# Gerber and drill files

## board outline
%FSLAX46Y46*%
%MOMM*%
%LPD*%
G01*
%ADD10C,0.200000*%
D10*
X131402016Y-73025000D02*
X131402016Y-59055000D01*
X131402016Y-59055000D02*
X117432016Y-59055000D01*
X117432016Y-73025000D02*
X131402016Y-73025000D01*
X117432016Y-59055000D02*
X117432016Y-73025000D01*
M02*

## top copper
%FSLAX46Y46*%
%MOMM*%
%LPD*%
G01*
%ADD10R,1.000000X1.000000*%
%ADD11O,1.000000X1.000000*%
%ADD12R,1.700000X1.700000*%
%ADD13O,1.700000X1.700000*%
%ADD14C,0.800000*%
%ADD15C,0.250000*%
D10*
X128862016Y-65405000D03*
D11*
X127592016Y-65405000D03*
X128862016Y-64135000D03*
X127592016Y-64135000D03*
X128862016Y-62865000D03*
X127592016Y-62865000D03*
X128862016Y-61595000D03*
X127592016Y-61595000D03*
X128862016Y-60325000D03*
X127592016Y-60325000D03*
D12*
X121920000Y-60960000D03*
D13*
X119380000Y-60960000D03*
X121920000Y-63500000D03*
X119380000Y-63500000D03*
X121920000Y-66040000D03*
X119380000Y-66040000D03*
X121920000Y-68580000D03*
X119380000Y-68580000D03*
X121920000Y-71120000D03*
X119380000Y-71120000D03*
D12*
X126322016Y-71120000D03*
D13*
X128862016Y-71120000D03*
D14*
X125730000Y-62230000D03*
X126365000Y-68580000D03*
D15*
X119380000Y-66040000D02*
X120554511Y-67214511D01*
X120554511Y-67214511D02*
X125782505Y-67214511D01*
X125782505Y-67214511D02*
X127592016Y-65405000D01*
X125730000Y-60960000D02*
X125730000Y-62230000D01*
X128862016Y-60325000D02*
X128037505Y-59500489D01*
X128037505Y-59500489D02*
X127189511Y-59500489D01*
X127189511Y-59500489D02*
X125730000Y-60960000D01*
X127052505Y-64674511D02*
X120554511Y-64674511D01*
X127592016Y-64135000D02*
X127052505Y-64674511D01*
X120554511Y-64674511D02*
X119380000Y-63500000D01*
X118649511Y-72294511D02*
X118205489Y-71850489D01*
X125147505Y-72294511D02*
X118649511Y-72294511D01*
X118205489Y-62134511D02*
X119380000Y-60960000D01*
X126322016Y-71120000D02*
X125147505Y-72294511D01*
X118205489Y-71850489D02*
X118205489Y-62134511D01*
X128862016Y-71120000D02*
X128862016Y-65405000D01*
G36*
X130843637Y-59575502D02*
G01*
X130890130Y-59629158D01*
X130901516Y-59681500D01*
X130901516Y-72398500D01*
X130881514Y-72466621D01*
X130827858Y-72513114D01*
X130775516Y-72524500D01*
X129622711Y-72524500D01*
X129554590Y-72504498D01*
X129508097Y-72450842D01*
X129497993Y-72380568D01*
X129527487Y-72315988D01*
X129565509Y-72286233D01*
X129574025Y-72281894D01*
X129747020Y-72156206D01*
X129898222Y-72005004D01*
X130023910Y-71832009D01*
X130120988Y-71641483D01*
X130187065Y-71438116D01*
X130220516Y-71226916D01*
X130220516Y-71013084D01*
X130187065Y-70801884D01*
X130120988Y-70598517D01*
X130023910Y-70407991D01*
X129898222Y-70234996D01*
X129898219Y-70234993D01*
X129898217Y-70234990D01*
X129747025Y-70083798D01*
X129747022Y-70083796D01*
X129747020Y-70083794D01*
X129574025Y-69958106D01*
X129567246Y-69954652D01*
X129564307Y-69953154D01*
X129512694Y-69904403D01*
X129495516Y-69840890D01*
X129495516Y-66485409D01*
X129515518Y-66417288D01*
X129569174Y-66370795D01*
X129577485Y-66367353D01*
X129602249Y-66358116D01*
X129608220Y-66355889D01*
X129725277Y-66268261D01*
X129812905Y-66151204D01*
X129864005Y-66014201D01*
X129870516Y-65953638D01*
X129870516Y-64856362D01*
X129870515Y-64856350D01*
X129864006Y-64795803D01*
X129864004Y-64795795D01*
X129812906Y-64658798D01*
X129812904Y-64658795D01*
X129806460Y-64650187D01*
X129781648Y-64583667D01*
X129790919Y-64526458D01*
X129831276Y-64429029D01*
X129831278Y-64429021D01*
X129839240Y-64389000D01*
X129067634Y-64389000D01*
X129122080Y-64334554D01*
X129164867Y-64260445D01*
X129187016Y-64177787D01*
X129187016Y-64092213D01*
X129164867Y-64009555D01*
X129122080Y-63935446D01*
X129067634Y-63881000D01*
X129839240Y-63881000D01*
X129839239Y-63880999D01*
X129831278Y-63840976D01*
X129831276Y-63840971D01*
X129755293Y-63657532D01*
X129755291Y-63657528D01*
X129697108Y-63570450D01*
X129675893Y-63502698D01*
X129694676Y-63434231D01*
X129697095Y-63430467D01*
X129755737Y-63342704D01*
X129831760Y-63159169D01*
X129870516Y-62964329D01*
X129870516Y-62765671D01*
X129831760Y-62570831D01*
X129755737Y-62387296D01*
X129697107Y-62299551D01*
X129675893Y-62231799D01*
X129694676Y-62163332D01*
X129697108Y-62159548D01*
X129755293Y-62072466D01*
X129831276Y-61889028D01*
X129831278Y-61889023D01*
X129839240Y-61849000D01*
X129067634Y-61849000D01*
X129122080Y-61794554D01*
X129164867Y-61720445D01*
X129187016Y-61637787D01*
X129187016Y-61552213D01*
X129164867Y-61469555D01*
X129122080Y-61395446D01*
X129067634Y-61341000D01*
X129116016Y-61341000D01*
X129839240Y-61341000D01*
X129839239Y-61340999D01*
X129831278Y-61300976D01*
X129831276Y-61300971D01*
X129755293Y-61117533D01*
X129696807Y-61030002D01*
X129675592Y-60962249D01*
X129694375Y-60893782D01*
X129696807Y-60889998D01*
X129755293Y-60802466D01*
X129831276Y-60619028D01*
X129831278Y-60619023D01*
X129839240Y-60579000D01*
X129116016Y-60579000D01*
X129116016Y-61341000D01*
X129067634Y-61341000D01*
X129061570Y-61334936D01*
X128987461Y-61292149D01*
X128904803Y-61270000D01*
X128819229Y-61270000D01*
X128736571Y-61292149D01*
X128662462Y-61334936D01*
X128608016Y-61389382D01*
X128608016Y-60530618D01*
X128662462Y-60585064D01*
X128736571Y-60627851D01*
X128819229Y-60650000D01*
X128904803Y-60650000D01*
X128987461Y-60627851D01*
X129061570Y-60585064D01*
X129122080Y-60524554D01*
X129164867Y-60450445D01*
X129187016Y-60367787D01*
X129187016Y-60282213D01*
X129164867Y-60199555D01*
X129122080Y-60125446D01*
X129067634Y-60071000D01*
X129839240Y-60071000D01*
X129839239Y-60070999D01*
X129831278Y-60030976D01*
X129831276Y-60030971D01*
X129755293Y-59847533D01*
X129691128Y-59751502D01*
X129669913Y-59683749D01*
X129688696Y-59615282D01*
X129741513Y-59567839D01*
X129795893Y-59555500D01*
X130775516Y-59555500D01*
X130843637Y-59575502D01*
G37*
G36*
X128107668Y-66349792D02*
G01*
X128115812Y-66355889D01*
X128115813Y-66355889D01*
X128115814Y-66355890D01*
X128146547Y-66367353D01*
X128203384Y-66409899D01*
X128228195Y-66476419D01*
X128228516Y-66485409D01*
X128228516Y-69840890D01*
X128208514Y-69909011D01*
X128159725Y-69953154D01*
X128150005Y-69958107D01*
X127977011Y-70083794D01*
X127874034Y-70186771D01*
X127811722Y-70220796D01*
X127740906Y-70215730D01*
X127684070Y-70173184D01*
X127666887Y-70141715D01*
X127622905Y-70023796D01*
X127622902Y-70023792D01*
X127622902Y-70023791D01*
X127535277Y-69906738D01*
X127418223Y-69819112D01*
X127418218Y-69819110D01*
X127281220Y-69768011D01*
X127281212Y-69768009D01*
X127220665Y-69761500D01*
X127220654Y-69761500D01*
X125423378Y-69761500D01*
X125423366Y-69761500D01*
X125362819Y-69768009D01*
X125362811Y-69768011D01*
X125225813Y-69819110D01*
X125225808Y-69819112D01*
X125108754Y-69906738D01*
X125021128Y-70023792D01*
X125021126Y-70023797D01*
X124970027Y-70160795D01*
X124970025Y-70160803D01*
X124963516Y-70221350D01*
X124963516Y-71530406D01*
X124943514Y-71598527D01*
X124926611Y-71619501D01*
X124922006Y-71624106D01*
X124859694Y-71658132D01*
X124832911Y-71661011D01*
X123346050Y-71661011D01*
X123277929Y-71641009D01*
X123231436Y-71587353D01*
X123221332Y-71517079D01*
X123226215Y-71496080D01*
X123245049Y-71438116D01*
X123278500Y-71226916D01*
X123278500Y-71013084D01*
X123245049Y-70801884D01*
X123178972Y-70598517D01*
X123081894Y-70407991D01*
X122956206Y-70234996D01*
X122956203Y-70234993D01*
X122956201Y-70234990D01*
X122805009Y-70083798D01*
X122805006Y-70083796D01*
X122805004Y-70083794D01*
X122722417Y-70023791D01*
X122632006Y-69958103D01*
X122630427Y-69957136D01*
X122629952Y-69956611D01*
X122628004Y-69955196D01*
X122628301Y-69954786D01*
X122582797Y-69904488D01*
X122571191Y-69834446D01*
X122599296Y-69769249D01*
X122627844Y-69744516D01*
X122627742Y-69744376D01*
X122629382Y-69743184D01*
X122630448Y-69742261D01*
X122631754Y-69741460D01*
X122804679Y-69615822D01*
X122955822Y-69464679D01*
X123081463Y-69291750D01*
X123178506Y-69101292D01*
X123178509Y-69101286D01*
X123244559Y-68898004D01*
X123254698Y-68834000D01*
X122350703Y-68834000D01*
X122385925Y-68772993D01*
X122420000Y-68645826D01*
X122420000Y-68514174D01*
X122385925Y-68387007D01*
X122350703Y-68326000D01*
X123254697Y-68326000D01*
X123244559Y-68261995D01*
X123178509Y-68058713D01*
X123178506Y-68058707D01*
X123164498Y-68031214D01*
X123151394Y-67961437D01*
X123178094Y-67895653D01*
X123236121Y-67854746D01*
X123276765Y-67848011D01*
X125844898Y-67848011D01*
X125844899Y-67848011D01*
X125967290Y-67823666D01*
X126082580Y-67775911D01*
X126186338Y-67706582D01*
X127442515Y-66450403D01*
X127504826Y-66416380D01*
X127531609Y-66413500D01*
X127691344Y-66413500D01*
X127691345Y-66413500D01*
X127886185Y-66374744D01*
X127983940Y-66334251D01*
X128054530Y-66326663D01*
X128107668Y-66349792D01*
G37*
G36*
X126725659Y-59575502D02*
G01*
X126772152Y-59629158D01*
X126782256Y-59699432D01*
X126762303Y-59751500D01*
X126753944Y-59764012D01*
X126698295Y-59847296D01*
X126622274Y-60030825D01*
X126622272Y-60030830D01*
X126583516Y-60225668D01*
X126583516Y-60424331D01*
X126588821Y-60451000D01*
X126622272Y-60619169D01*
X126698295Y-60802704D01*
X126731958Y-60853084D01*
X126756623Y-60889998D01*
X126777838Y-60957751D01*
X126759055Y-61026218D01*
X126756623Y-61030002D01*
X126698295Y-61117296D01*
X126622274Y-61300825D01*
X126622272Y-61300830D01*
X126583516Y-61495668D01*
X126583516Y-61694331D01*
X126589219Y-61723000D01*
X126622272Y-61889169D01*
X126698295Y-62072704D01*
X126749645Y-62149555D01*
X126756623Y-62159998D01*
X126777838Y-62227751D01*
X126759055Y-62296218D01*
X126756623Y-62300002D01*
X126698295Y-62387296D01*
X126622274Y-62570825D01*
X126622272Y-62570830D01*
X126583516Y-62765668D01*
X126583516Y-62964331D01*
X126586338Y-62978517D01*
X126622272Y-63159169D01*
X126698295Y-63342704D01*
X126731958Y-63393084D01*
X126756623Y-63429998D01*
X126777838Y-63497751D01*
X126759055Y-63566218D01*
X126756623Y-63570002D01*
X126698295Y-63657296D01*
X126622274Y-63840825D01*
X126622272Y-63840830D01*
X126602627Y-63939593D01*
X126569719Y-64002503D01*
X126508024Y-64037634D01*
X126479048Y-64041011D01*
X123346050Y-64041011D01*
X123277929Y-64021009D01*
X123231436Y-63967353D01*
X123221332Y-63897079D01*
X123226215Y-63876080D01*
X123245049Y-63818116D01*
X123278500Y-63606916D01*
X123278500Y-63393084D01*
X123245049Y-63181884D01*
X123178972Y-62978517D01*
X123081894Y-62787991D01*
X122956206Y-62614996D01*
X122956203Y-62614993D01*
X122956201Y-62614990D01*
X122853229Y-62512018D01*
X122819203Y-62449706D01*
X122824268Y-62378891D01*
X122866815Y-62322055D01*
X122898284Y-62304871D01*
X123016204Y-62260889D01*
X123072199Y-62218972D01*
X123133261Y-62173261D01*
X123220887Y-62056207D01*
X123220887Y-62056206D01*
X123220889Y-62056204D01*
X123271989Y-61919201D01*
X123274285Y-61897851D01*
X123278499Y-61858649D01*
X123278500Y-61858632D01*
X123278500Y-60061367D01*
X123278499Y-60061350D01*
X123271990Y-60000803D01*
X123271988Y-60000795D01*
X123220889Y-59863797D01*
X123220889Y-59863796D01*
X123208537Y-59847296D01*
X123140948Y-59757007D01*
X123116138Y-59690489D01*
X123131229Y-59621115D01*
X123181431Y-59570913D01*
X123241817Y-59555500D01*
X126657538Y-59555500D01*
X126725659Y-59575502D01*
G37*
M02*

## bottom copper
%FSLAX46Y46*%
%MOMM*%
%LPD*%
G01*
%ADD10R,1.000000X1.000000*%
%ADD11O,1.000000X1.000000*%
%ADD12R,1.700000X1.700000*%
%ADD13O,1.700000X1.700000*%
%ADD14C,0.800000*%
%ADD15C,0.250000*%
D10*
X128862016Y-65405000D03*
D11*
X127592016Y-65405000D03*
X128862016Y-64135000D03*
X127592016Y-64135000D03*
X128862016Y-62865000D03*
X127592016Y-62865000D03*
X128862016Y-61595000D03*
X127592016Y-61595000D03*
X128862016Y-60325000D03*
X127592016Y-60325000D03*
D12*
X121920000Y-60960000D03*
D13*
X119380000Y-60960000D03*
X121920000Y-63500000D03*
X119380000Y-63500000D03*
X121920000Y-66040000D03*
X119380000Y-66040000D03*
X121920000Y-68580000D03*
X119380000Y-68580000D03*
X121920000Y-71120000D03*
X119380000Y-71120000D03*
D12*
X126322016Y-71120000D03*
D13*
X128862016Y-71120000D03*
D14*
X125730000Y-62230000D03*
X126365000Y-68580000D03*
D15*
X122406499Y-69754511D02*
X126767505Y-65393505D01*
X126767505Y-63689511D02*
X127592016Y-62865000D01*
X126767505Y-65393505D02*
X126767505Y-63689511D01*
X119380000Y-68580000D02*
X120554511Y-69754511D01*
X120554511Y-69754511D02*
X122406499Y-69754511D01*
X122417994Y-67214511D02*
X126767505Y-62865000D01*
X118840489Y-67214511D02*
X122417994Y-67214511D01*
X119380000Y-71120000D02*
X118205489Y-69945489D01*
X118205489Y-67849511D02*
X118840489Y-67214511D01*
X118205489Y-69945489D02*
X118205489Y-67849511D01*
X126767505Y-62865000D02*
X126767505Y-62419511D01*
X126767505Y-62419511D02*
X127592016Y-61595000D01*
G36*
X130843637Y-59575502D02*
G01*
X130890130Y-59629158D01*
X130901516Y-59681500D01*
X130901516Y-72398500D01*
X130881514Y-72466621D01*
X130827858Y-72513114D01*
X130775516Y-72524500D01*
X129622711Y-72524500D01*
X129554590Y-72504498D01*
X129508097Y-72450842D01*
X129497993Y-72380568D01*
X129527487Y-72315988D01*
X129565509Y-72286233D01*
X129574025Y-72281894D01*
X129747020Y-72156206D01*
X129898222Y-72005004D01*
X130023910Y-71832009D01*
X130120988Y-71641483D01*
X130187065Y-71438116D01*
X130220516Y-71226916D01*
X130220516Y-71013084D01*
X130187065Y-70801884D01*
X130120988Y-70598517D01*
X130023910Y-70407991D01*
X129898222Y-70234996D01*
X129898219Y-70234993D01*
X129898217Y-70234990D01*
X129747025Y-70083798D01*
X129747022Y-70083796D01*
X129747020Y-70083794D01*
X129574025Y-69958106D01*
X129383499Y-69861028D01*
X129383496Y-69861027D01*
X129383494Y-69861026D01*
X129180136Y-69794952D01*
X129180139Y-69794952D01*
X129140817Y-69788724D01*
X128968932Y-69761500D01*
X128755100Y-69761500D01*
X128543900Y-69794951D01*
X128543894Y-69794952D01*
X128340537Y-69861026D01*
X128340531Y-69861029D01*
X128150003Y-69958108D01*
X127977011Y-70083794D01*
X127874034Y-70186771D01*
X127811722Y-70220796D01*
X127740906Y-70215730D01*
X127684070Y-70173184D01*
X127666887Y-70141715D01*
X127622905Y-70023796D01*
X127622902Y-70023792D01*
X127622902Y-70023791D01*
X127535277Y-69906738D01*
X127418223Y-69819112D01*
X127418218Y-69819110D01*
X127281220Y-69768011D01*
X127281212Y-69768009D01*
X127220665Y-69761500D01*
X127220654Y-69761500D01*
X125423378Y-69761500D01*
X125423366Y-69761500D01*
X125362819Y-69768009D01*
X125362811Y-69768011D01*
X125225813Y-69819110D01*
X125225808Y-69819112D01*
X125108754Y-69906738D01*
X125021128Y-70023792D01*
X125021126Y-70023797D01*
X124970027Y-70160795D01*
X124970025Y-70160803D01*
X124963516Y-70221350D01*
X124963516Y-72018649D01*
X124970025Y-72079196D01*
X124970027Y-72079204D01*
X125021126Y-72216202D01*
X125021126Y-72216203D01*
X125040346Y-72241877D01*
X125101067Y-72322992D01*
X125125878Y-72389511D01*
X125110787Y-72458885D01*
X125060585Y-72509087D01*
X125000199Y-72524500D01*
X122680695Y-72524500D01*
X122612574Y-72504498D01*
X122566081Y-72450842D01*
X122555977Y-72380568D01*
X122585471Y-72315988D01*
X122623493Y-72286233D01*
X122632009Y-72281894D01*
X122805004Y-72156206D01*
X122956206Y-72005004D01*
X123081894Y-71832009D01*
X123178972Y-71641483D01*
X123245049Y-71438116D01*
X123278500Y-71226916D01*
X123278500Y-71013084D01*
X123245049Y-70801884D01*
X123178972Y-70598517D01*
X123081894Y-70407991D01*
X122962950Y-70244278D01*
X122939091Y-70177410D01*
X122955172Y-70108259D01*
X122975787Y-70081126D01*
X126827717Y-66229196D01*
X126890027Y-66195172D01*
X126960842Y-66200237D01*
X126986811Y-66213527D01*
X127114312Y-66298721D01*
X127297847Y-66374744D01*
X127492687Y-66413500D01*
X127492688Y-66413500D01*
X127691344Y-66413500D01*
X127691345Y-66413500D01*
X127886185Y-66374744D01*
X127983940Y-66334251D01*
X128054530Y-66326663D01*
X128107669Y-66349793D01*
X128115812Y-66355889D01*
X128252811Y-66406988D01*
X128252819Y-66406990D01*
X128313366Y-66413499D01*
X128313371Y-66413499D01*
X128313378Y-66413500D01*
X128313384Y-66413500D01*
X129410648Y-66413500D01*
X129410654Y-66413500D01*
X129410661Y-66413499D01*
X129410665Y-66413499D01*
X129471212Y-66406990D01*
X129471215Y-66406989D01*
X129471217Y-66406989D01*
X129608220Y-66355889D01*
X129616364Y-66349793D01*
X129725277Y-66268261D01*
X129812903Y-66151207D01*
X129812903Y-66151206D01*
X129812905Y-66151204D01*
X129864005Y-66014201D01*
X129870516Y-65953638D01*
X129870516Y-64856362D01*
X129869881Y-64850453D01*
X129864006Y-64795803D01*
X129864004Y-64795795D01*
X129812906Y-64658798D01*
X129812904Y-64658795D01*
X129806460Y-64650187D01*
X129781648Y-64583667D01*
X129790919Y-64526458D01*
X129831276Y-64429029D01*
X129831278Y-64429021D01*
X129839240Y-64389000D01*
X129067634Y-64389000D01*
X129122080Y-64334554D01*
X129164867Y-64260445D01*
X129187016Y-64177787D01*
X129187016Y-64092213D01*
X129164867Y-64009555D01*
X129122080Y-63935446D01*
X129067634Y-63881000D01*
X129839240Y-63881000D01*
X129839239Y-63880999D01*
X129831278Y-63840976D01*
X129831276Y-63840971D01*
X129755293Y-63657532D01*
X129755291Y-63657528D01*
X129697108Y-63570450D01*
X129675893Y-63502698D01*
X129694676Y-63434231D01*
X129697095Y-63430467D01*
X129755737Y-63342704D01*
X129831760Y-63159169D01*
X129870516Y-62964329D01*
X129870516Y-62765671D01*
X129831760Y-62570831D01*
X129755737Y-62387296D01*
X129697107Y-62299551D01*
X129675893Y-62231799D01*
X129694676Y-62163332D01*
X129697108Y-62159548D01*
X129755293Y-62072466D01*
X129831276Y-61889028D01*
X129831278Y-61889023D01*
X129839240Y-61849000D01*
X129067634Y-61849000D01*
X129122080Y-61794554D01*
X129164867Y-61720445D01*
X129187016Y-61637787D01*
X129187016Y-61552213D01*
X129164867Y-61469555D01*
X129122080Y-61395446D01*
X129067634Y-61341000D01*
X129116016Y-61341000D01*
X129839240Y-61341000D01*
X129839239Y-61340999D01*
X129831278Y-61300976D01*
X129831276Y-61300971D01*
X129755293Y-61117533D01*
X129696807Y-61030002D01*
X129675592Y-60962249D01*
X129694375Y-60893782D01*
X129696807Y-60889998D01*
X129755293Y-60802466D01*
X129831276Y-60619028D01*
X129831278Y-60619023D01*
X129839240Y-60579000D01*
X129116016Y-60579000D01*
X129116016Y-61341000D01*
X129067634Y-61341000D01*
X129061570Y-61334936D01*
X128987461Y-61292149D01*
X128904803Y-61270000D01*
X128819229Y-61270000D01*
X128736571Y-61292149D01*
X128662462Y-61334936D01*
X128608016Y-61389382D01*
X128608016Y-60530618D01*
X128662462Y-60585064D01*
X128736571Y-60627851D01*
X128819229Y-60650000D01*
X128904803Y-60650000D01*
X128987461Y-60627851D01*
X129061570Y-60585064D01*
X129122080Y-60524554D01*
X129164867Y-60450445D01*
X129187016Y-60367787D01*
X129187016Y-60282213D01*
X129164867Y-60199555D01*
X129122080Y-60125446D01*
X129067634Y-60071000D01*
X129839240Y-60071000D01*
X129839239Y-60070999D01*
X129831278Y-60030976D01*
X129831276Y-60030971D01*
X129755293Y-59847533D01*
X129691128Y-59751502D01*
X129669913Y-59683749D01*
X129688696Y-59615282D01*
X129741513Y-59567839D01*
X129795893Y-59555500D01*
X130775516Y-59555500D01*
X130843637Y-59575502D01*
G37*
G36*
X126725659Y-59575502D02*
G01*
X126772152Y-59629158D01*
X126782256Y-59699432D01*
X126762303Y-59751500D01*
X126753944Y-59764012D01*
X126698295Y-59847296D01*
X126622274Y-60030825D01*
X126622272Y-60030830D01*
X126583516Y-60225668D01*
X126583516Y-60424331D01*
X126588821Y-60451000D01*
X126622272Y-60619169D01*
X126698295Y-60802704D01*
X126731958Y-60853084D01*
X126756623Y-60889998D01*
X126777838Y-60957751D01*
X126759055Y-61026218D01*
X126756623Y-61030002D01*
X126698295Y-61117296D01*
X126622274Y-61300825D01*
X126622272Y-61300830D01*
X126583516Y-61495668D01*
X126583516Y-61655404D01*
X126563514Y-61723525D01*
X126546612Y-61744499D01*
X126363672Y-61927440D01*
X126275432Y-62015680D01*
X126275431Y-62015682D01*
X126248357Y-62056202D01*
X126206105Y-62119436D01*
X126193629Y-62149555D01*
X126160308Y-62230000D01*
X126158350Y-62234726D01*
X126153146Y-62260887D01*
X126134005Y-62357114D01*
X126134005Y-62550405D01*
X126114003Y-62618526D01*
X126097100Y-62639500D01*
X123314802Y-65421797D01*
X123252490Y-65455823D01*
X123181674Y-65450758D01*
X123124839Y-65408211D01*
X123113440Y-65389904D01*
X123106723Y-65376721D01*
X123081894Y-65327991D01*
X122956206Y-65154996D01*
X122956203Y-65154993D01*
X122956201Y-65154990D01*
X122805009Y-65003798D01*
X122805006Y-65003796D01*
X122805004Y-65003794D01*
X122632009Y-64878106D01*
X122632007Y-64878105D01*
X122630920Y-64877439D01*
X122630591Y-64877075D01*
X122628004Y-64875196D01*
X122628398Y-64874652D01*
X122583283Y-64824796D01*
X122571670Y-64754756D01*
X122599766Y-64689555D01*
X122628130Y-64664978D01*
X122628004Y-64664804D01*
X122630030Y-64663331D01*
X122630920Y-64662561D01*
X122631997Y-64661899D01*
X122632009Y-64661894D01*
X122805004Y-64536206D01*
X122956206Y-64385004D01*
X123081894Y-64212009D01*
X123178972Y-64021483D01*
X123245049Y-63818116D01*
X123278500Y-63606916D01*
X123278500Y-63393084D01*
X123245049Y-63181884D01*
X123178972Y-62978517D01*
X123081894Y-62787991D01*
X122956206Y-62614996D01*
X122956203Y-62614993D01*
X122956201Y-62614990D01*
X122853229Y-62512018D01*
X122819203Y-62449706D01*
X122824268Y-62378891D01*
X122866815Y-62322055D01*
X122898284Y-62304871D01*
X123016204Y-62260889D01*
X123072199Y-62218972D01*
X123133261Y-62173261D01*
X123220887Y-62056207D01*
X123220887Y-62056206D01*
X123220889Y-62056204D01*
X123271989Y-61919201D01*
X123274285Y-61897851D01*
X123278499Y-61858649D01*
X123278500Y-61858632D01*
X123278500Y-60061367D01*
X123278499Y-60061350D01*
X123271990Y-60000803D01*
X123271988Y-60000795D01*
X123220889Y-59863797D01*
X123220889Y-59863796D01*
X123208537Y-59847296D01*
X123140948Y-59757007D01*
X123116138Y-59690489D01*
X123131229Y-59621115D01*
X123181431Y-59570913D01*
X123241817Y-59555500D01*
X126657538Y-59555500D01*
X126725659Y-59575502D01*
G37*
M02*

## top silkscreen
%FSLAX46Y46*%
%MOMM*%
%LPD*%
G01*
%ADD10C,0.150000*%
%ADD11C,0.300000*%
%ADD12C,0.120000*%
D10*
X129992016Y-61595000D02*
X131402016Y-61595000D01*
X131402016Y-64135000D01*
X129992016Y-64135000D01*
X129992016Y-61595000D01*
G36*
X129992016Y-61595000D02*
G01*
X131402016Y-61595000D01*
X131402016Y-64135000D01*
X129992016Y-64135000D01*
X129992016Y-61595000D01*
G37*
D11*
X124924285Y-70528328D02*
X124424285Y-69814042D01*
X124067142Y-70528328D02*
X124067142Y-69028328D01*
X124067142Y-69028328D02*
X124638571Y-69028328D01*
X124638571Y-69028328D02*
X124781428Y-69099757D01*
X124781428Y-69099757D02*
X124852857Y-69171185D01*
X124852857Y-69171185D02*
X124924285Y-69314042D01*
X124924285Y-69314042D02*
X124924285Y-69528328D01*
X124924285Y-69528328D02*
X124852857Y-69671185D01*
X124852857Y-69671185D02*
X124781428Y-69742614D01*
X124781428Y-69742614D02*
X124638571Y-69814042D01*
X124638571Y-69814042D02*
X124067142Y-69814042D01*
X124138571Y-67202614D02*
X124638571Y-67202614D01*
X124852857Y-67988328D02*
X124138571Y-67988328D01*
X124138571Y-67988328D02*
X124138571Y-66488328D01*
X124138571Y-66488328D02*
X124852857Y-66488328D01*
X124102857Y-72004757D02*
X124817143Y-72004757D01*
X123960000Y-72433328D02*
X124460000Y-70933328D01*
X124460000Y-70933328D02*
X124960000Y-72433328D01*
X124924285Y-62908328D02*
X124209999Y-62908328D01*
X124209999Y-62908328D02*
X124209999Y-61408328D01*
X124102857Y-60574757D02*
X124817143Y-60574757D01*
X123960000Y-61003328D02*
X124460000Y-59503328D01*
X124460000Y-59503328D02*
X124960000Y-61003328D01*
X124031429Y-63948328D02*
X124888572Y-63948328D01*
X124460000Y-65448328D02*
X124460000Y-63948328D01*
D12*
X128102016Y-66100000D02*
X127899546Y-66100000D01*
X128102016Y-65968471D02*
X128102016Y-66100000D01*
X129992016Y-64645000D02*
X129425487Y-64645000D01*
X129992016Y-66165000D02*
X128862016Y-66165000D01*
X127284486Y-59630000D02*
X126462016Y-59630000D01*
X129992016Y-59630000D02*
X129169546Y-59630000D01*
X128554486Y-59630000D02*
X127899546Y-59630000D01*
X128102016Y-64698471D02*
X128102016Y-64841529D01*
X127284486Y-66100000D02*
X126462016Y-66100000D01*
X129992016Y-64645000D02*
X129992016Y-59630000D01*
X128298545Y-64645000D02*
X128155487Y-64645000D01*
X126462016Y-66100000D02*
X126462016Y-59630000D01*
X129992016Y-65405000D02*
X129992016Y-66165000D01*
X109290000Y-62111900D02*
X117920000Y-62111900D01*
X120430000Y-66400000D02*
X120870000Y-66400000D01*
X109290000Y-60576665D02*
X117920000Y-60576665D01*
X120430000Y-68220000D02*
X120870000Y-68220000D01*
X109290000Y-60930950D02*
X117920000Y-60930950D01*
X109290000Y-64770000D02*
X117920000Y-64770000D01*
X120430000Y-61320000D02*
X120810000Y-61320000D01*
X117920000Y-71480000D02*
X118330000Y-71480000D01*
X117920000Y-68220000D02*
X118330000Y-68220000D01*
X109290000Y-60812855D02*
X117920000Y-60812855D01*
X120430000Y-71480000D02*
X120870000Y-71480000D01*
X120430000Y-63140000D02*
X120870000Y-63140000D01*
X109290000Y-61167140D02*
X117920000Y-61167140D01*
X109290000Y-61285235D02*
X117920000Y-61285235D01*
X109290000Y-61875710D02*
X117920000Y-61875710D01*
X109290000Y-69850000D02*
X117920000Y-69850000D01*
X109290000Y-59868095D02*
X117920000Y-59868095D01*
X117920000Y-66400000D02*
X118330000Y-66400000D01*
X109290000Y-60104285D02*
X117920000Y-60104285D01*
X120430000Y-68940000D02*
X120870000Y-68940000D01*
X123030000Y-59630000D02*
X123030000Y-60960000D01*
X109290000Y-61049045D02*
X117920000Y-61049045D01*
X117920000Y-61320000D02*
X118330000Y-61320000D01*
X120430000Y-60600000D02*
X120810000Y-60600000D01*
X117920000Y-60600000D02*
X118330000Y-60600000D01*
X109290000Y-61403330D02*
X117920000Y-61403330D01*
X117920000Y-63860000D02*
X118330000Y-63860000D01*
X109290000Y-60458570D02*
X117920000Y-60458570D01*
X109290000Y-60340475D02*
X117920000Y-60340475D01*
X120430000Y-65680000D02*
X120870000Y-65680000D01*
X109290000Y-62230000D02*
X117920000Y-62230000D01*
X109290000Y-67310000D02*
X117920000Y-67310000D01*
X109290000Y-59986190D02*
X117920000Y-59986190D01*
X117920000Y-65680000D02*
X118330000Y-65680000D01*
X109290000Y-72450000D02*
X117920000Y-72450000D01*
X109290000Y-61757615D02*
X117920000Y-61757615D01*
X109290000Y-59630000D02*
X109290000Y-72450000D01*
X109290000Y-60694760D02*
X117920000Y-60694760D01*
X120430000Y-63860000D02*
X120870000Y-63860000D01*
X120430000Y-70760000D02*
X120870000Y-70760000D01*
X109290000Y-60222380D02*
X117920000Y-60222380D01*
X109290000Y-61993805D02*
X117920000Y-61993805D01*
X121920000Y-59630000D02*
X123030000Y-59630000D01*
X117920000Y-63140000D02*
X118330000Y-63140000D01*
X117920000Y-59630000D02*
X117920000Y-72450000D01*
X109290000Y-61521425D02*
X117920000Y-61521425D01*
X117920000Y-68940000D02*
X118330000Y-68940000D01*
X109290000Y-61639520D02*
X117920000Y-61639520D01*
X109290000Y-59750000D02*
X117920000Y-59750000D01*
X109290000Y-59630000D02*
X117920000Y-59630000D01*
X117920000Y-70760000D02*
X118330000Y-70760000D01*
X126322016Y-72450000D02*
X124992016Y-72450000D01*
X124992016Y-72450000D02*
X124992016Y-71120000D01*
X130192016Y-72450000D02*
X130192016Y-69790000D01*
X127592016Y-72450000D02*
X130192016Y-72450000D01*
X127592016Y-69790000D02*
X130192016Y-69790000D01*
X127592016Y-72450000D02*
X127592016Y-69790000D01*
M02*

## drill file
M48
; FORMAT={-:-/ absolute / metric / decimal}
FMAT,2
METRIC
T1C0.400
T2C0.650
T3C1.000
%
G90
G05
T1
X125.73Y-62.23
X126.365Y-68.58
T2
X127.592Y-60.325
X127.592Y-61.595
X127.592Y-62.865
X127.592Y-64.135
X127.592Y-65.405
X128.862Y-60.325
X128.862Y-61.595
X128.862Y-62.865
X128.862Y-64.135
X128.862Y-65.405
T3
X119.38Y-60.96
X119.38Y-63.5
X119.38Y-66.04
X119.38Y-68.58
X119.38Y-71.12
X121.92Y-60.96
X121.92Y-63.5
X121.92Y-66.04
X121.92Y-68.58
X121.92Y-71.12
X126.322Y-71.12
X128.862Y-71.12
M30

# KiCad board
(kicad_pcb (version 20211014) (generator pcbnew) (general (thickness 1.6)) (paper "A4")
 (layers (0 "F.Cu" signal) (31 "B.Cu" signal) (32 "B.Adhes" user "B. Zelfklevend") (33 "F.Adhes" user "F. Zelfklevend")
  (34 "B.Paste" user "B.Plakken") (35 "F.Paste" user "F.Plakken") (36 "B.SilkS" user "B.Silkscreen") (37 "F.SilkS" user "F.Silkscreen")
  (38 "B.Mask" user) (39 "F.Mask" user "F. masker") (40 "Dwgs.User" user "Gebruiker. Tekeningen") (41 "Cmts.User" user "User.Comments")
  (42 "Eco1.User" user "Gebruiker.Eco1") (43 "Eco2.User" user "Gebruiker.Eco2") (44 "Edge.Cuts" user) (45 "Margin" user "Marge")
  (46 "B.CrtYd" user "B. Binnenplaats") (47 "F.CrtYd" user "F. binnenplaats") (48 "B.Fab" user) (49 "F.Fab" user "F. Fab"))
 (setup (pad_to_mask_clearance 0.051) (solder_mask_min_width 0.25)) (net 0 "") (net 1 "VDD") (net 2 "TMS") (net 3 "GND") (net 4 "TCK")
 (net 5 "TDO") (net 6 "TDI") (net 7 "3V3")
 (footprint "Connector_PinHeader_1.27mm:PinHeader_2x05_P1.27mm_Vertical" (layer "F.Cu") (at 128.862016 65.405 180)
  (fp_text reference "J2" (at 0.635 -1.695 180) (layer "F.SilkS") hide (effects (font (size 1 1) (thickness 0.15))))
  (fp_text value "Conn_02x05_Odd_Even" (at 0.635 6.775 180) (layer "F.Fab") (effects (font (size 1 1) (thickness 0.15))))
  (fp_line (start 0.76 -0.695) (end 0.96247 -0.695) (layer "F.SilkS") (width 0.12))
  (fp_line (start 0.76 -0.563471) (end 0.76 -0.695) (layer "F.SilkS") (width 0.12))
  (fp_line (start -1.13 0.76) (end -0.563471 0.76) (layer "F.SilkS") (width 0.12))
  (fp_line (start -1.13 -0.76) (end 0 -0.76) (layer "F.SilkS") (width 0.12))
  (fp_line (start 1.57753 5.775) (end 2.4 5.775) (layer "F.SilkS") (width 0.12))
  (fp_line (start -1.13 5.775) (end -0.30753 5.775) (layer "F.SilkS") (width 0.12))
  (fp_line (start 0.30753 5.775) (end 0.96247 5.775) (layer "F.SilkS") (width 0.12))
  (fp_line (start 0.76 0.706529) (end 0.76 0.563471) (layer "F.SilkS") (width 0.12))
  (fp_line (start 1.57753 -0.695) (end 2.4 -0.695) (layer "F.SilkS") (width 0.12))
  (fp_line (start -1.13 0.76) (end -1.13 5.775) (layer "F.SilkS") (width 0.12))
  (fp_line (start 0.563471 0.76) (end 0.706529 0.76) (layer "F.SilkS") (width 0.12))
  (fp_line (start 2.4 -0.695) (end 2.4 5.775) (layer "F.SilkS") (width 0.12))
  (fp_line (start -1.13 0) (end -1.13 -0.76) (layer "F.SilkS") (width 0.12))
  (pad "1" thru_hole rect locked (at 0 0 180) (size 1 1) (drill 0.65) (layers *.Cu *.Mask) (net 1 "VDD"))
  (pad "2" thru_hole oval locked (at 1.27 0 180) (size 1 1) (drill 0.65) (layers *.Cu *.Mask) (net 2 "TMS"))
  (pad "3" thru_hole oval locked (at 0 1.27 180) (size 1 1) (drill 0.65) (layers *.Cu *.Mask) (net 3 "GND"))
  (pad "4" thru_hole oval locked (at 1.27 1.27 180) (size 1 1) (drill 0.65) (layers *.Cu *.Mask) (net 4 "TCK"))
  (pad "5" thru_hole oval locked (at 0 2.54 180) (size 1 1) (drill 0.65) (layers *.Cu *.Mask))
  (pad "6" thru_hole oval locked (at 1.27 2.54 180) (size 1 1) (drill 0.65) (layers *.Cu *.Mask) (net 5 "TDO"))
  (pad "7" thru_hole oval locked (at 0 3.81 180) (size 1 1) (drill 0.65) (layers *.Cu *.Mask) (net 3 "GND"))
  (pad "8" thru_hole oval locked (at 1.27 3.81 180) (size 1 1) (drill 0.65) (layers *.Cu *.Mask) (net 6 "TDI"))
  (pad "9" thru_hole oval locked (at 0 5.08 180) (size 1 1) (drill 0.65) (layers *.Cu *.Mask) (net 3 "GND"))
  (pad "10" thru_hole oval locked (at 1.27 5.08 180) (size 1 1) (drill 0.65) (layers *.Cu *.Mask)))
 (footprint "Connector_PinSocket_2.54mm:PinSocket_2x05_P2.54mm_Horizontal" (layer "F.Cu") (at 121.92 60.96)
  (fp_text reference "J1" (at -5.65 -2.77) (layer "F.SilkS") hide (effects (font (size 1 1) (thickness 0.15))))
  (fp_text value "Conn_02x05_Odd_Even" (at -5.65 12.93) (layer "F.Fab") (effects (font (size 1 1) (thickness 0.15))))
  (fp_line (start -12.63 1.1519) (end -4 1.1519) (layer "F.SilkS") (width 0.12))
  (fp_line (start -1.49 5.44) (end -1.05 5.44) (layer "F.SilkS") (width 0.12))
  (fp_line (start -12.63 -0.383335) (end -4 -0.383335) (layer "F.SilkS") (width 0.12))
  (fp_line (start -1.49 7.26) (end -1.05 7.26) (layer "F.SilkS") (width 0.12))
  (fp_line (start -12.63 -0.02905) (end -4 -0.02905) (layer "F.SilkS") (width 0.12))
  (fp_line (start -12.63 3.81) (end -4 3.81) (layer "F.SilkS") (width 0.12))
  (fp_line (start -1.49 0.36) (end -1.11 0.36) (layer "F.SilkS") (width 0.12))
  (fp_line (start -4 10.52) (end -3.59 10.52) (layer "F.SilkS") (width 0.12))
  (fp_line (start -4 7.26) (end -3.59 7.26) (layer "F.SilkS") (width 0.12))
  (fp_line (start -12.63 -0.147145) (end -4 -0.147145) (layer "F.SilkS") (width 0.12))
  (fp_line (start -1.49 10.52) (end -1.05 10.52) (layer "F.SilkS") (width 0.12))
  (fp_line (start -1.49 2.18) (end -1.05 2.18) (layer "F.SilkS") (width 0.12))
  (fp_line (start -12.63 0.20714) (end -4 0.20714) (layer "F.SilkS") (width 0.12))
  (fp_line (start -12.63 0.325235) (end -4 0.325235) (layer "F.SilkS") (width 0.12))
  (fp_line (start -12.63 0.91571) (end -4 0.91571) (layer "F.SilkS") (width 0.12))
  (fp_line (start -12.63 8.89) (end -4 8.89) (layer "F.SilkS") (width 0.12))
  (fp_line (start -12.63 -1.091905) (end -4 -1.091905) (layer "F.SilkS") (width 0.12))
  (fp_line (start -4 5.44) (end -3.59 5.44) (layer "F.SilkS") (width 0.12))
  (fp_line (start -12.63 -0.855715) (end -4 -0.855715) (layer "F.SilkS") (width 0.12))
  (fp_line (start -1.49 7.98) (end -1.05 7.98) (layer "F.SilkS") (width 0.12))
  (fp_line (start 1.11 -1.33) (end 1.11 0) (layer "F.SilkS") (width 0.12))
  (fp_line (start -12.63 0.089045) (end -4 0.089045) (layer "F.SilkS") (width 0.12))
  (fp_line (start -4 0.36) (end -3.59 0.36) (layer "F.SilkS") (width 0.12))
  (fp_line (start -1.49 -0.36) (end -1.11 -0.36) (layer "F.SilkS") (width 0.12))
  (fp_line (start -4 -0.36) (end -3.59 -0.36) (layer "F.SilkS") (width 0.12))
  (fp_line (start -12.63 0.44333) (end -4 0.44333) (layer "F.SilkS") (width 0.12))
  (fp_line (start -4 2.9) (end -3.59 2.9) (layer "F.SilkS") (width 0.12))
  (fp_line (start -12.63 -0.50143) (end -4 -0.50143) (layer "F.SilkS") (width 0.12))
  (fp_line (start -12.63 -0.619525) (end -4 -0.619525) (layer "F.SilkS") (width 0.12))
  (fp_line (start -1.49 4.72) (end -1.05 4.72) (layer "F.SilkS") (width 0.12))
  (fp_line (start -12.63 1.27) (end -4 1.27) (layer "F.SilkS") (width 0.12))
  (fp_line (start -12.63 6.35) (end -4 6.35) (layer "F.SilkS") (width 0.12))
  (fp_line (start -12.63 -0.97381) (end -4 -0.97381) (layer "F.SilkS") (width 0.12))
  (fp_line (start -4 4.72) (end -3.59 4.72) (layer "F.SilkS") (width 0.12))
  (fp_line (start -12.63 11.49) (end -4 11.49) (layer "F.SilkS") (width 0.12))
  (fp_line (start -12.63 0.797615) (end -4 0.797615) (layer "F.SilkS") (width 0.12))
  (fp_line (start -12.63 -1.33) (end -12.63 11.49) (layer "F.SilkS") (width 0.12))
  (fp_line (start -12.63 -0.26524) (end -4 -0.26524) (layer "F.SilkS") (width 0.12))
  (fp_line (start -1.49 2.9) (end -1.05 2.9) (layer "F.SilkS") (width 0.12))
  (fp_line (start -1.49 9.8) (end -1.05 9.8) (layer "F.SilkS") (width 0.12))
  (fp_line (start -12.63 -0.73762) (end -4 -0.73762) (layer "F.SilkS") (width 0.12))
  (fp_line (start -12.63 1.033805) (end -4 1.033805) (layer "F.SilkS") (width 0.12))
  (fp_line (start 0 -1.33) (end 1.11 -1.33) (layer "F.SilkS") (width 0.12))
  (fp_line (start -4 2.18) (end -3.59 2.18) (layer "F.SilkS") (width 0.12))
  (fp_line (start -4 -1.33) (end -4 11.49) (layer "F.SilkS") (width 0.12))
  (fp_line (start -12.63 0.561425) (end -4 0.561425) (layer "F.SilkS") (width 0.12))
  (fp_line (start -4 7.98) (end -3.59 7.98) (layer "F.SilkS") (width 0.12))
  (fp_line (start -12.63 0.67952) (end -4 0.67952) (layer "F.SilkS") (width 0.12))
  (fp_line (start -12.63 -1.21) (end -4 -1.21) (layer "F.SilkS") (width 0.12))
  (fp_line (start -12.63 -1.33) (end -4 -1.33) (layer "F.SilkS") (width 0.12))
  (fp_line (start -4 9.8) (end -3.59 9.8) (layer "F.SilkS") (width 0.12))
  (pad "1" thru_hole rect locked (at 0 0) (size 1.7 1.7) (drill 1) (layers *.Cu *.Mask))
  (pad "2" thru_hole oval locked (at -2.54 0) (size 1.7 1.7) (drill 1) (layers *.Cu *.Mask) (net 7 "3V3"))
  (pad "3" thru_hole oval locked (at 0 2.54) (size 1.7 1.7) (drill 1) (layers *.Cu *.Mask))
  (pad "4" thru_hole oval locked (at -2.54 2.54) (size 1.7 1.7) (drill 1) (layers *.Cu *.Mask) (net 4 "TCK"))
  (pad "5" thru_hole oval locked (at 0 5.08) (size 1.7 1.7) (drill 1) (layers *.Cu *.Mask))
  (pad "6" thru_hole oval locked (at -2.54 5.08) (size 1.7 1.7) (drill 1) (layers *.Cu *.Mask) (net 2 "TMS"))
  (pad "7" thru_hole oval locked (at 0 7.62) (size 1.7 1.7) (drill 1) (layers *.Cu *.Mask) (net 3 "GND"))
  (pad "8" thru_hole oval locked (at -2.54 7.62) (size 1.7 1.7) (drill 1) (layers *.Cu *.Mask) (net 5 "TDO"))
  (pad "9" thru_hole oval locked (at 0 10.16) (size 1.7 1.7) (drill 1) (layers *.Cu *.Mask))
  (pad "10" thru_hole oval locked (at -2.54 10.16) (size 1.7 1.7) (drill 1) (layers *.Cu *.Mask) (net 6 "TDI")))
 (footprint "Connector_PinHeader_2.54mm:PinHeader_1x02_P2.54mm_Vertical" (layer "F.Cu") (at 126.322016 71.12 90)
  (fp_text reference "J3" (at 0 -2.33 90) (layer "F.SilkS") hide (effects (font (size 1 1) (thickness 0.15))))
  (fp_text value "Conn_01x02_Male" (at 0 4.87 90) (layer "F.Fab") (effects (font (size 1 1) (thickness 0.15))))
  (fp_line (start -1.33 0) (end -1.33 -1.33) (layer "F.SilkS") (width 0.12))
  (fp_line (start -1.33 -1.33) (end 0 -1.33) (layer "F.SilkS") (width 0.12))
  (fp_line (start -1.33 3.87) (end 1.33 3.87) (layer "F.SilkS") (width 0.12))
  (fp_line (start -1.33 1.27) (end -1.33 3.87) (layer "F.SilkS") (width 0.12))
  (fp_line (start 1.33 1.27) (end 1.33 3.87) (layer "F.SilkS") (width 0.12))
  (fp_line (start -1.33 1.27) (end 1.33 1.27) (layer "F.SilkS") (width 0.12))
  (pad "1" thru_hole rect locked (at 0 0 90) (size 1.7 1.7) (drill 1) (layers *.Cu *.Mask) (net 7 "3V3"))
  (pad "2" thru_hole oval locked (at 0 2.54 90) (size 1.7 1.7) (drill 1) (layers *.Cu *.Mask) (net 1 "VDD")))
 (gr_rect (start 129.992016 61.595) (end 131.402016 64.135) (layer "F.SilkS") (width 0.15) (fill solid))
 (gr_line (start 131.402016 73.025) (end 131.402016 59.055) (layer "Edge.Cuts") (width 0.2))
 (gr_line (start 131.402016 59.055) (end 117.432016 59.055) (layer "Edge.Cuts") (width 0.2))
 (gr_line (start 117.432016 73.025) (end 131.402016 73.025) (layer "Edge.Cuts") (width 0.2))
 (gr_line (start 117.432016 59.055) (end 117.432016 73.025) (layer "Edge.Cuts") (width 0.2))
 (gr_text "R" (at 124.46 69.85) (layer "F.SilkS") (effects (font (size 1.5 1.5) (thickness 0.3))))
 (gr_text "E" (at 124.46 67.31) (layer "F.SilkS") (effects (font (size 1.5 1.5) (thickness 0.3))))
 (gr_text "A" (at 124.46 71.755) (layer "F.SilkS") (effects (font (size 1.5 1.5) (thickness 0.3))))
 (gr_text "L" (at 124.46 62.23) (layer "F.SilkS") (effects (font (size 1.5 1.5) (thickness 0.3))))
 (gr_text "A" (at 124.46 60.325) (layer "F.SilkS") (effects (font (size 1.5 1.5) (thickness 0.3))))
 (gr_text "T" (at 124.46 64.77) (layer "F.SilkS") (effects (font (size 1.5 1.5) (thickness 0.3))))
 (segment (start 119.38 66.04) (end 120.554511 67.214511) (width 0.25) (layer "F.Cu") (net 2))
 (segment (start 120.554511 67.214511) (end 125.782505 67.214511) (width 0.25) (layer "F.Cu") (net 2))
 (segment (start 125.782505 67.214511) (end 127.592016 65.405) (width 0.25) (layer "F.Cu") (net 2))
 (segment (start 125.73 60.96) (end 125.73 62.23) (width 0.25) (layer "F.Cu") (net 3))
 (segment (start 128.862016 60.325) (end 128.037505 59.500489) (width 0.25) (layer "F.Cu") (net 3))
 (segment (start 128.037505 59.500489) (end 127.189511 59.500489) (width 0.25) (layer "F.Cu") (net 3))
 (segment (start 127.189511 59.500489) (end 125.73 60.96) (width 0.25) (layer "F.Cu") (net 3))
 (via (at 125.73 62.23) (size 0.8) (drill 0.4) (layers "F.Cu" "B.Cu") (free) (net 3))
 (via (at 126.365 68.58) (size 0.8) (drill 0.4) (layers "F.Cu" "B.Cu") (free) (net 3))
 (segment (start 127.052505 64.674511) (end 120.554511 64.674511) (width 0.25) (layer "F.Cu") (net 4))
 (segment (start 127.592016 64.135) (end 127.052505 64.674511) (width 0.25) (layer "F.Cu") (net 4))
 (segment (start 120.554511 64.674511) (end 119.38 63.5) (width 0.25) (layer "F.Cu") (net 4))
 (segment (start 118.649511 72.294511) (end 118.205489 71.850489) (width 0.25) (layer "F.Cu") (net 7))
 (segment (start 125.147505 72.294511) (end 118.649511 72.294511) (width 0.25) (layer "F.Cu") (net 7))
 (segment (start 118.205489 62.134511) (end 119.38 60.96) (width 0.25) (layer "F.Cu") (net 7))
 (segment (start 126.322016 71.12) (end 125.147505 72.294511) (width 0.25) (layer "F.Cu") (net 7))
 (segment (start 118.205489 71.850489) (end 118.205489 62.134511) (width 0.25) (layer "F.Cu") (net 7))
 (segment (start 128.862016 71.12) (end 128.862016 65.405) (width 0.25) (layer "F.Cu") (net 1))
 (segment (start 122.406499 69.754511) (end 126.767505 65.393505) (width 0.25) (layer "B.Cu") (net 5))
 (segment (start 126.767505 63.689511) (end 127.592016 62.865) (width 0.25) (layer "B.Cu") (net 5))
 (segment (start 126.767505 65.393505) (end 126.767505 63.689511) (width 0.25) (layer "B.Cu") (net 5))
 (segment (start 119.38 68.58) (end 120.554511 69.754511) (width 0.25) (layer "B.Cu") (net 5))
 (segment (start 120.554511 69.754511) (end 122.406499 69.754511) (width 0.25) (layer "B.Cu") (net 5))
 (segment (start 122.417994 67.214511) (end 126.767505 62.865) (width 0.25) (layer "B.Cu") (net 6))
 (segment (start 118.840489 67.214511) (end 122.417994 67.214511) (width 0.25) (layer "B.Cu") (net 6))
 (segment (start 119.38 71.12) (end 118.205489 69.945489) (width 0.25) (layer "B.Cu") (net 6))
 (segment (start 118.205489 67.849511) (end 118.840489 67.214511) (width 0.25) (layer "B.Cu") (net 6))
 (segment (start 118.205489 69.945489) (end 118.205489 67.849511) (width 0.25) (layer "B.Cu") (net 6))
 (segment (start 126.767505 62.865) (end 126.767505 62.419511) (width 0.25) (layer "B.Cu") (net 6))
 (segment (start 126.767505 62.419511) (end 127.592016 61.595) (width 0.25) (layer "B.Cu") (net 6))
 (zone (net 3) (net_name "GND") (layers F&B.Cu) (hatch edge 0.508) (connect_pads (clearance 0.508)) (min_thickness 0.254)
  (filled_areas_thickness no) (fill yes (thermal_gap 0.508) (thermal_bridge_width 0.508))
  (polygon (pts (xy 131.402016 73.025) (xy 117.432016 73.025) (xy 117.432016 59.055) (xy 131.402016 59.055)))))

